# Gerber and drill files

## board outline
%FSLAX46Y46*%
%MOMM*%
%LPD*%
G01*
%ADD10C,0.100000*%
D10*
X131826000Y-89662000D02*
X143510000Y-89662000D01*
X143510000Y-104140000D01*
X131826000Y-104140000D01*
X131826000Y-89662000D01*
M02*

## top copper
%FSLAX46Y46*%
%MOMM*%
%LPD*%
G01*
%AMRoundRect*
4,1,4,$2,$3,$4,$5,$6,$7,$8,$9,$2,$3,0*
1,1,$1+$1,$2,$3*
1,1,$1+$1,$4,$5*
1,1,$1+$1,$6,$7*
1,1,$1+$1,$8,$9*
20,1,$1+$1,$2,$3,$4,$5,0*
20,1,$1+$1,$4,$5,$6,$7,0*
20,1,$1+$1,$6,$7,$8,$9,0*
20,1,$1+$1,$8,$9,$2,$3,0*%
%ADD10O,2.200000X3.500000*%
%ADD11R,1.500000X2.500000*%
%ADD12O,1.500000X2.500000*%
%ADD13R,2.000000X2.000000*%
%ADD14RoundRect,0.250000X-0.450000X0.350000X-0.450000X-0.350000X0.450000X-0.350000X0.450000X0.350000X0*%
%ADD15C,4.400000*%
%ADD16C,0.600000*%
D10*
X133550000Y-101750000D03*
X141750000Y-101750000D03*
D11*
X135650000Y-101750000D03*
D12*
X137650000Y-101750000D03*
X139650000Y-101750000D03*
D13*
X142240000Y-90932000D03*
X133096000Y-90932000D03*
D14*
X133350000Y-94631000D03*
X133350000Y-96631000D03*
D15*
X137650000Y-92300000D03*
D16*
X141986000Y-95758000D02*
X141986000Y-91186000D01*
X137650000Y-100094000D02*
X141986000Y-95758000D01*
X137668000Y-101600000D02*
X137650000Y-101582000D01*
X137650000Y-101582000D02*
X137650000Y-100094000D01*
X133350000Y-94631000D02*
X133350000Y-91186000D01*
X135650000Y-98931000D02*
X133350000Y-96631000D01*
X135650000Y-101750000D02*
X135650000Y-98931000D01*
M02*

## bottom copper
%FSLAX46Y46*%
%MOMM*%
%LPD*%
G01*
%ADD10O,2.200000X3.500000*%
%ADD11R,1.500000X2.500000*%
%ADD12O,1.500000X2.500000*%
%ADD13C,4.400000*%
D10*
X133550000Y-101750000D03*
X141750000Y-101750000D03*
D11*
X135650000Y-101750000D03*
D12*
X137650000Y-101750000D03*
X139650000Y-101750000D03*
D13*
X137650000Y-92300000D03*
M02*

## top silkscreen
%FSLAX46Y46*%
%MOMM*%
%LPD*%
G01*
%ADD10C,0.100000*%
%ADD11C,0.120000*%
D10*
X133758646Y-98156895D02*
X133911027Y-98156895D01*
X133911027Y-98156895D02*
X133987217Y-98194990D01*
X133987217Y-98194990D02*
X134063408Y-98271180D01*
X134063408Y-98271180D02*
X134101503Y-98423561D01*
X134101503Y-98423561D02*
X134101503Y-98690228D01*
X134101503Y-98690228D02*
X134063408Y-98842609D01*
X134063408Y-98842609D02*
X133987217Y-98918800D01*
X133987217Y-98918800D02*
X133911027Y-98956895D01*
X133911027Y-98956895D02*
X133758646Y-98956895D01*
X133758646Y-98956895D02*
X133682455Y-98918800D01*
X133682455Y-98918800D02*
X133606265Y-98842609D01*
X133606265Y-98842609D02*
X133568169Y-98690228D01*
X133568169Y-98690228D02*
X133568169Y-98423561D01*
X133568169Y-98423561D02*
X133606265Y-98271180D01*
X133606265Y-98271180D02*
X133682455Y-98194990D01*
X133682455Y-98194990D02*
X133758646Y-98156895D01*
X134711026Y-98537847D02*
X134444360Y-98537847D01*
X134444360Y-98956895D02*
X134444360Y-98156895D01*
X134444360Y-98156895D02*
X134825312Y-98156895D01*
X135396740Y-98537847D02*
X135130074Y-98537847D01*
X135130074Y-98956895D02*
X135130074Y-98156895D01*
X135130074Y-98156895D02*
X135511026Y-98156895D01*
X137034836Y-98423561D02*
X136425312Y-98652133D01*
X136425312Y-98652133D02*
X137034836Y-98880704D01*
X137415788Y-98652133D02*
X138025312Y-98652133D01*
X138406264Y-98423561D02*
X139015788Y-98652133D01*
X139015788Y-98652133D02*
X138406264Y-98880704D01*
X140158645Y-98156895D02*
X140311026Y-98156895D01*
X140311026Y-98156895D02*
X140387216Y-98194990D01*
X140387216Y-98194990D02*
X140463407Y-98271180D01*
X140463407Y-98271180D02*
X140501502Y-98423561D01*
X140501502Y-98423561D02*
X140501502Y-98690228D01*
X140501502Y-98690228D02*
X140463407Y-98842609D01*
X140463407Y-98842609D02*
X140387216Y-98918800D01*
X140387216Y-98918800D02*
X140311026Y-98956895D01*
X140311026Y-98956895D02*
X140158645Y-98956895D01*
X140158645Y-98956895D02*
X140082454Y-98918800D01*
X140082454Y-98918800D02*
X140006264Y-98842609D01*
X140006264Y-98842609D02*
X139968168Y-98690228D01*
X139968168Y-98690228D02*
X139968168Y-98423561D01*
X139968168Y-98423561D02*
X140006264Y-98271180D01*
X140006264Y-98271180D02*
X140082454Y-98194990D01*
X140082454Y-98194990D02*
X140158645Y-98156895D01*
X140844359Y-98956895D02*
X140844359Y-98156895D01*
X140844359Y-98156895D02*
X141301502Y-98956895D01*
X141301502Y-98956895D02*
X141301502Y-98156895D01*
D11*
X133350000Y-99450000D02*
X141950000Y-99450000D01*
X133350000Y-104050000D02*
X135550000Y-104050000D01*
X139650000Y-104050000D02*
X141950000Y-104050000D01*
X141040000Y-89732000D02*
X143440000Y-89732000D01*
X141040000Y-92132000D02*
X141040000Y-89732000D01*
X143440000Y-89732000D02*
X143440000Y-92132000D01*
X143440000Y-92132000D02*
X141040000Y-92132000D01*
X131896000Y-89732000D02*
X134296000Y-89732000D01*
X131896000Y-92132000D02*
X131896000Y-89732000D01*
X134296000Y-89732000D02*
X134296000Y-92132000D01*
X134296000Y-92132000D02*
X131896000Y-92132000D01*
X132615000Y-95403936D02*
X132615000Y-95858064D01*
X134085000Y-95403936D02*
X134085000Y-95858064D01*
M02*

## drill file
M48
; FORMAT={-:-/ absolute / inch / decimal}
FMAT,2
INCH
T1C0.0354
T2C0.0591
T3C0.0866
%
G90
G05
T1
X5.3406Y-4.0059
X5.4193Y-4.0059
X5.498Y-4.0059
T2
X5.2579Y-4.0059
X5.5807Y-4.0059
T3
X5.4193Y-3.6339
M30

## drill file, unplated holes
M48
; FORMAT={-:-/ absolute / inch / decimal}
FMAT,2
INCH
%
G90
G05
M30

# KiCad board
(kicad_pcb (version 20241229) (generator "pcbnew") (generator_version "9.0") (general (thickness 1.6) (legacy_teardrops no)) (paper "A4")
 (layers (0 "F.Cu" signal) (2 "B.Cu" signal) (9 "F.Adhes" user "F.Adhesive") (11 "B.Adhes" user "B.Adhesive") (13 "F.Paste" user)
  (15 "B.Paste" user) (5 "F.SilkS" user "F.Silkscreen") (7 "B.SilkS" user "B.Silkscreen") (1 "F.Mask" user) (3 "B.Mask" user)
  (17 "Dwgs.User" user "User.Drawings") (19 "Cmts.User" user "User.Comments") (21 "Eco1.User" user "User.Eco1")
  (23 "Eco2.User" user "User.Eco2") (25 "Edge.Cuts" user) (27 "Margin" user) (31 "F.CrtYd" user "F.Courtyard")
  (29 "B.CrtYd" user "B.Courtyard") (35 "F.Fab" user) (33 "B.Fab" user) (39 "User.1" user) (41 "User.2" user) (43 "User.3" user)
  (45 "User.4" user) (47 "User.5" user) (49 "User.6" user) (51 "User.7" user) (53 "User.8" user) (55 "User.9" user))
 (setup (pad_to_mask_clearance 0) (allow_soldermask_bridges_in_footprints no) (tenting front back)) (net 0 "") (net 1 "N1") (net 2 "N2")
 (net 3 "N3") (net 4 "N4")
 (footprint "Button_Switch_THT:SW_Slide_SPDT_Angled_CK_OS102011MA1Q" (layer "F.Cu") (at 135.65 101.75)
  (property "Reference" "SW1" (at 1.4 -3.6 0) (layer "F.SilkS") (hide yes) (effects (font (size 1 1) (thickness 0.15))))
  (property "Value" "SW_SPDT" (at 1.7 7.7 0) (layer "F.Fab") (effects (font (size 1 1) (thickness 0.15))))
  (fp_line (start -2.3 -2.3) (end 6.3 -2.3) (stroke (width 0.12) (type solid)) (layer "F.SilkS"))
  (fp_line (start -2.3 2.3) (end -0.1 2.3) (stroke (width 0.12) (type solid)) (layer "F.SilkS"))
  (fp_line (start 4 2.3) (end 6.3 2.3) (stroke (width 0.12) (type solid)) (layer "F.SilkS"))
  (pad "" thru_hole oval (at -2.1 0) (size 2.2 3.5) (drill 1.5) (layers "*.Cu" "*.Mask") (remove_unused_layers no))
  (pad "" thru_hole oval (at 6.1 0) (size 2.2 3.5) (drill 1.5) (layers "*.Cu" "*.Mask") (remove_unused_layers no))
  (pad "1" thru_hole rect (at 0 0) (size 1.5 2.5) (drill 0.9) (layers "*.Cu" "*.Mask") (remove_unused_layers no) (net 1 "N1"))
  (pad "2" thru_hole oval (at 2 0) (size 1.5 2.5) (drill 0.9) (layers "*.Cu" "*.Mask") (remove_unused_layers no) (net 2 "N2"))
  (pad "3" thru_hole oval (at 4 0) (size 1.5 2.5) (drill 0.9) (layers "*.Cu" "*.Mask") (remove_unused_layers no) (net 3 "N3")))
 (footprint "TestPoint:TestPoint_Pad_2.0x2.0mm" (layer "F.Cu") (at 142.24 90.932)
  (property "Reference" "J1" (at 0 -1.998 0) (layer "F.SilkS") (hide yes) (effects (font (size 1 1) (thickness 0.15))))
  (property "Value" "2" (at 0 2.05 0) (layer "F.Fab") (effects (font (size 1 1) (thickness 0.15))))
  (fp_line (start -1.2 -1.2) (end 1.2 -1.2) (stroke (width 0.12) (type solid)) (layer "F.SilkS"))
  (fp_line (start -1.2 1.2) (end -1.2 -1.2) (stroke (width 0.12) (type solid)) (layer "F.SilkS"))
  (fp_line (start 1.2 -1.2) (end 1.2 1.2) (stroke (width 0.12) (type solid)) (layer "F.SilkS"))
  (fp_line (start 1.2 1.2) (end -1.2 1.2) (stroke (width 0.12) (type solid)) (layer "F.SilkS"))
  (pad "1" smd rect (at 0 0) (size 2 2) (layers "F.Cu" "F.Mask") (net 2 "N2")))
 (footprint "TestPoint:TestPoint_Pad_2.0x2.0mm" (layer "F.Cu") (at 133.096 90.932)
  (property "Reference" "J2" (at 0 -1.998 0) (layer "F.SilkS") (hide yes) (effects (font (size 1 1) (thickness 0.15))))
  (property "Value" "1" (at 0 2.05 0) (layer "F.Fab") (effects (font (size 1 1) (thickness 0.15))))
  (fp_line (start -1.2 -1.2) (end 1.2 -1.2) (stroke (width 0.12) (type solid)) (layer "F.SilkS"))
  (fp_line (start -1.2 1.2) (end -1.2 -1.2) (stroke (width 0.12) (type solid)) (layer "F.SilkS"))
  (fp_line (start 1.2 -1.2) (end 1.2 1.2) (stroke (width 0.12) (type solid)) (layer "F.SilkS"))
  (fp_line (start 1.2 1.2) (end -1.2 1.2) (stroke (width 0.12) (type solid)) (layer "F.SilkS"))
  (pad "1" smd rect (at 0 0) (size 2 2) (layers "F.Cu" "F.Mask") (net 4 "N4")))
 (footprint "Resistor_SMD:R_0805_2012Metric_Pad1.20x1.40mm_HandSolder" (layer "F.Cu") (at 133.35 95.631 -90)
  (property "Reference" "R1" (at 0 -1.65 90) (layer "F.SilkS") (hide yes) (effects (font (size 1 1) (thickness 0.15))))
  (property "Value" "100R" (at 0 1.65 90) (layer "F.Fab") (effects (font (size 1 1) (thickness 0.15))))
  (fp_line (start -0.227064 0.735) (end 0.227064 0.735) (stroke (width 0.12) (type solid)) (layer "F.SilkS"))
  (fp_line (start -0.227064 -0.735) (end 0.227064 -0.735) (stroke (width 0.12) (type solid)) (layer "F.SilkS"))
  (pad "1" smd roundrect (at -1 0 270) (size 1.2 1.4) (layers "F.Cu" "F.Mask" "F.Paste") (roundrect_rratio 0.2083333333) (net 4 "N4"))
  (pad "2" smd roundrect (at 1 0 270) (size 1.2 1.4) (layers "F.Cu" "F.Mask" "F.Paste") (roundrect_rratio 0.2083333333) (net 1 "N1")))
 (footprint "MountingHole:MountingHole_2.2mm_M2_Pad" (layer "F.Cu") (at 137.65 92.3)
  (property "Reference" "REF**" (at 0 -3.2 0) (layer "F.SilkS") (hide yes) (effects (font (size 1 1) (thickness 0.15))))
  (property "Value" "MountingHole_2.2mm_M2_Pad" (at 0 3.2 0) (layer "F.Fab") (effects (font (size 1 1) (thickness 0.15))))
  (pad "1" thru_hole circle (at 0 0) (size 4.4 4.4) (drill 2.2) (layers "*.Cu" "*.Mask") (remove_unused_layers no)))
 (gr_rect (start 131.826 89.662) (end 143.51 104.14) (stroke (width 0.1) (type default)) (fill no) (layer "Edge.Cuts"))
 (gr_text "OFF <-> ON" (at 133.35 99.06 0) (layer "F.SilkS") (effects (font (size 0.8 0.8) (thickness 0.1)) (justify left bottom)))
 (segment (start 141.986 95.758) (end 141.986 91.186) (width 0.6) (layer "F.Cu") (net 2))
 (segment (start 137.65 100.094) (end 141.986 95.758) (width 0.6) (layer "F.Cu") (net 2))
 (segment (start 137.668 101.6) (end 137.65 101.582) (width 0.6) (layer "F.Cu") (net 2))
 (segment (start 137.65 101.582) (end 137.65 100.094) (width 0.6) (layer "F.Cu") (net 2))
 (segment (start 133.35 94.631) (end 133.35 91.186) (width 0.6) (layer "F.Cu") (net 4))
 (segment (start 135.65 98.931) (end 133.35 96.631) (width 0.6) (layer "F.Cu") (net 1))
 (segment (start 135.65 101.75) (end 135.65 98.931) (width 0.6) (layer "F.Cu") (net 1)))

